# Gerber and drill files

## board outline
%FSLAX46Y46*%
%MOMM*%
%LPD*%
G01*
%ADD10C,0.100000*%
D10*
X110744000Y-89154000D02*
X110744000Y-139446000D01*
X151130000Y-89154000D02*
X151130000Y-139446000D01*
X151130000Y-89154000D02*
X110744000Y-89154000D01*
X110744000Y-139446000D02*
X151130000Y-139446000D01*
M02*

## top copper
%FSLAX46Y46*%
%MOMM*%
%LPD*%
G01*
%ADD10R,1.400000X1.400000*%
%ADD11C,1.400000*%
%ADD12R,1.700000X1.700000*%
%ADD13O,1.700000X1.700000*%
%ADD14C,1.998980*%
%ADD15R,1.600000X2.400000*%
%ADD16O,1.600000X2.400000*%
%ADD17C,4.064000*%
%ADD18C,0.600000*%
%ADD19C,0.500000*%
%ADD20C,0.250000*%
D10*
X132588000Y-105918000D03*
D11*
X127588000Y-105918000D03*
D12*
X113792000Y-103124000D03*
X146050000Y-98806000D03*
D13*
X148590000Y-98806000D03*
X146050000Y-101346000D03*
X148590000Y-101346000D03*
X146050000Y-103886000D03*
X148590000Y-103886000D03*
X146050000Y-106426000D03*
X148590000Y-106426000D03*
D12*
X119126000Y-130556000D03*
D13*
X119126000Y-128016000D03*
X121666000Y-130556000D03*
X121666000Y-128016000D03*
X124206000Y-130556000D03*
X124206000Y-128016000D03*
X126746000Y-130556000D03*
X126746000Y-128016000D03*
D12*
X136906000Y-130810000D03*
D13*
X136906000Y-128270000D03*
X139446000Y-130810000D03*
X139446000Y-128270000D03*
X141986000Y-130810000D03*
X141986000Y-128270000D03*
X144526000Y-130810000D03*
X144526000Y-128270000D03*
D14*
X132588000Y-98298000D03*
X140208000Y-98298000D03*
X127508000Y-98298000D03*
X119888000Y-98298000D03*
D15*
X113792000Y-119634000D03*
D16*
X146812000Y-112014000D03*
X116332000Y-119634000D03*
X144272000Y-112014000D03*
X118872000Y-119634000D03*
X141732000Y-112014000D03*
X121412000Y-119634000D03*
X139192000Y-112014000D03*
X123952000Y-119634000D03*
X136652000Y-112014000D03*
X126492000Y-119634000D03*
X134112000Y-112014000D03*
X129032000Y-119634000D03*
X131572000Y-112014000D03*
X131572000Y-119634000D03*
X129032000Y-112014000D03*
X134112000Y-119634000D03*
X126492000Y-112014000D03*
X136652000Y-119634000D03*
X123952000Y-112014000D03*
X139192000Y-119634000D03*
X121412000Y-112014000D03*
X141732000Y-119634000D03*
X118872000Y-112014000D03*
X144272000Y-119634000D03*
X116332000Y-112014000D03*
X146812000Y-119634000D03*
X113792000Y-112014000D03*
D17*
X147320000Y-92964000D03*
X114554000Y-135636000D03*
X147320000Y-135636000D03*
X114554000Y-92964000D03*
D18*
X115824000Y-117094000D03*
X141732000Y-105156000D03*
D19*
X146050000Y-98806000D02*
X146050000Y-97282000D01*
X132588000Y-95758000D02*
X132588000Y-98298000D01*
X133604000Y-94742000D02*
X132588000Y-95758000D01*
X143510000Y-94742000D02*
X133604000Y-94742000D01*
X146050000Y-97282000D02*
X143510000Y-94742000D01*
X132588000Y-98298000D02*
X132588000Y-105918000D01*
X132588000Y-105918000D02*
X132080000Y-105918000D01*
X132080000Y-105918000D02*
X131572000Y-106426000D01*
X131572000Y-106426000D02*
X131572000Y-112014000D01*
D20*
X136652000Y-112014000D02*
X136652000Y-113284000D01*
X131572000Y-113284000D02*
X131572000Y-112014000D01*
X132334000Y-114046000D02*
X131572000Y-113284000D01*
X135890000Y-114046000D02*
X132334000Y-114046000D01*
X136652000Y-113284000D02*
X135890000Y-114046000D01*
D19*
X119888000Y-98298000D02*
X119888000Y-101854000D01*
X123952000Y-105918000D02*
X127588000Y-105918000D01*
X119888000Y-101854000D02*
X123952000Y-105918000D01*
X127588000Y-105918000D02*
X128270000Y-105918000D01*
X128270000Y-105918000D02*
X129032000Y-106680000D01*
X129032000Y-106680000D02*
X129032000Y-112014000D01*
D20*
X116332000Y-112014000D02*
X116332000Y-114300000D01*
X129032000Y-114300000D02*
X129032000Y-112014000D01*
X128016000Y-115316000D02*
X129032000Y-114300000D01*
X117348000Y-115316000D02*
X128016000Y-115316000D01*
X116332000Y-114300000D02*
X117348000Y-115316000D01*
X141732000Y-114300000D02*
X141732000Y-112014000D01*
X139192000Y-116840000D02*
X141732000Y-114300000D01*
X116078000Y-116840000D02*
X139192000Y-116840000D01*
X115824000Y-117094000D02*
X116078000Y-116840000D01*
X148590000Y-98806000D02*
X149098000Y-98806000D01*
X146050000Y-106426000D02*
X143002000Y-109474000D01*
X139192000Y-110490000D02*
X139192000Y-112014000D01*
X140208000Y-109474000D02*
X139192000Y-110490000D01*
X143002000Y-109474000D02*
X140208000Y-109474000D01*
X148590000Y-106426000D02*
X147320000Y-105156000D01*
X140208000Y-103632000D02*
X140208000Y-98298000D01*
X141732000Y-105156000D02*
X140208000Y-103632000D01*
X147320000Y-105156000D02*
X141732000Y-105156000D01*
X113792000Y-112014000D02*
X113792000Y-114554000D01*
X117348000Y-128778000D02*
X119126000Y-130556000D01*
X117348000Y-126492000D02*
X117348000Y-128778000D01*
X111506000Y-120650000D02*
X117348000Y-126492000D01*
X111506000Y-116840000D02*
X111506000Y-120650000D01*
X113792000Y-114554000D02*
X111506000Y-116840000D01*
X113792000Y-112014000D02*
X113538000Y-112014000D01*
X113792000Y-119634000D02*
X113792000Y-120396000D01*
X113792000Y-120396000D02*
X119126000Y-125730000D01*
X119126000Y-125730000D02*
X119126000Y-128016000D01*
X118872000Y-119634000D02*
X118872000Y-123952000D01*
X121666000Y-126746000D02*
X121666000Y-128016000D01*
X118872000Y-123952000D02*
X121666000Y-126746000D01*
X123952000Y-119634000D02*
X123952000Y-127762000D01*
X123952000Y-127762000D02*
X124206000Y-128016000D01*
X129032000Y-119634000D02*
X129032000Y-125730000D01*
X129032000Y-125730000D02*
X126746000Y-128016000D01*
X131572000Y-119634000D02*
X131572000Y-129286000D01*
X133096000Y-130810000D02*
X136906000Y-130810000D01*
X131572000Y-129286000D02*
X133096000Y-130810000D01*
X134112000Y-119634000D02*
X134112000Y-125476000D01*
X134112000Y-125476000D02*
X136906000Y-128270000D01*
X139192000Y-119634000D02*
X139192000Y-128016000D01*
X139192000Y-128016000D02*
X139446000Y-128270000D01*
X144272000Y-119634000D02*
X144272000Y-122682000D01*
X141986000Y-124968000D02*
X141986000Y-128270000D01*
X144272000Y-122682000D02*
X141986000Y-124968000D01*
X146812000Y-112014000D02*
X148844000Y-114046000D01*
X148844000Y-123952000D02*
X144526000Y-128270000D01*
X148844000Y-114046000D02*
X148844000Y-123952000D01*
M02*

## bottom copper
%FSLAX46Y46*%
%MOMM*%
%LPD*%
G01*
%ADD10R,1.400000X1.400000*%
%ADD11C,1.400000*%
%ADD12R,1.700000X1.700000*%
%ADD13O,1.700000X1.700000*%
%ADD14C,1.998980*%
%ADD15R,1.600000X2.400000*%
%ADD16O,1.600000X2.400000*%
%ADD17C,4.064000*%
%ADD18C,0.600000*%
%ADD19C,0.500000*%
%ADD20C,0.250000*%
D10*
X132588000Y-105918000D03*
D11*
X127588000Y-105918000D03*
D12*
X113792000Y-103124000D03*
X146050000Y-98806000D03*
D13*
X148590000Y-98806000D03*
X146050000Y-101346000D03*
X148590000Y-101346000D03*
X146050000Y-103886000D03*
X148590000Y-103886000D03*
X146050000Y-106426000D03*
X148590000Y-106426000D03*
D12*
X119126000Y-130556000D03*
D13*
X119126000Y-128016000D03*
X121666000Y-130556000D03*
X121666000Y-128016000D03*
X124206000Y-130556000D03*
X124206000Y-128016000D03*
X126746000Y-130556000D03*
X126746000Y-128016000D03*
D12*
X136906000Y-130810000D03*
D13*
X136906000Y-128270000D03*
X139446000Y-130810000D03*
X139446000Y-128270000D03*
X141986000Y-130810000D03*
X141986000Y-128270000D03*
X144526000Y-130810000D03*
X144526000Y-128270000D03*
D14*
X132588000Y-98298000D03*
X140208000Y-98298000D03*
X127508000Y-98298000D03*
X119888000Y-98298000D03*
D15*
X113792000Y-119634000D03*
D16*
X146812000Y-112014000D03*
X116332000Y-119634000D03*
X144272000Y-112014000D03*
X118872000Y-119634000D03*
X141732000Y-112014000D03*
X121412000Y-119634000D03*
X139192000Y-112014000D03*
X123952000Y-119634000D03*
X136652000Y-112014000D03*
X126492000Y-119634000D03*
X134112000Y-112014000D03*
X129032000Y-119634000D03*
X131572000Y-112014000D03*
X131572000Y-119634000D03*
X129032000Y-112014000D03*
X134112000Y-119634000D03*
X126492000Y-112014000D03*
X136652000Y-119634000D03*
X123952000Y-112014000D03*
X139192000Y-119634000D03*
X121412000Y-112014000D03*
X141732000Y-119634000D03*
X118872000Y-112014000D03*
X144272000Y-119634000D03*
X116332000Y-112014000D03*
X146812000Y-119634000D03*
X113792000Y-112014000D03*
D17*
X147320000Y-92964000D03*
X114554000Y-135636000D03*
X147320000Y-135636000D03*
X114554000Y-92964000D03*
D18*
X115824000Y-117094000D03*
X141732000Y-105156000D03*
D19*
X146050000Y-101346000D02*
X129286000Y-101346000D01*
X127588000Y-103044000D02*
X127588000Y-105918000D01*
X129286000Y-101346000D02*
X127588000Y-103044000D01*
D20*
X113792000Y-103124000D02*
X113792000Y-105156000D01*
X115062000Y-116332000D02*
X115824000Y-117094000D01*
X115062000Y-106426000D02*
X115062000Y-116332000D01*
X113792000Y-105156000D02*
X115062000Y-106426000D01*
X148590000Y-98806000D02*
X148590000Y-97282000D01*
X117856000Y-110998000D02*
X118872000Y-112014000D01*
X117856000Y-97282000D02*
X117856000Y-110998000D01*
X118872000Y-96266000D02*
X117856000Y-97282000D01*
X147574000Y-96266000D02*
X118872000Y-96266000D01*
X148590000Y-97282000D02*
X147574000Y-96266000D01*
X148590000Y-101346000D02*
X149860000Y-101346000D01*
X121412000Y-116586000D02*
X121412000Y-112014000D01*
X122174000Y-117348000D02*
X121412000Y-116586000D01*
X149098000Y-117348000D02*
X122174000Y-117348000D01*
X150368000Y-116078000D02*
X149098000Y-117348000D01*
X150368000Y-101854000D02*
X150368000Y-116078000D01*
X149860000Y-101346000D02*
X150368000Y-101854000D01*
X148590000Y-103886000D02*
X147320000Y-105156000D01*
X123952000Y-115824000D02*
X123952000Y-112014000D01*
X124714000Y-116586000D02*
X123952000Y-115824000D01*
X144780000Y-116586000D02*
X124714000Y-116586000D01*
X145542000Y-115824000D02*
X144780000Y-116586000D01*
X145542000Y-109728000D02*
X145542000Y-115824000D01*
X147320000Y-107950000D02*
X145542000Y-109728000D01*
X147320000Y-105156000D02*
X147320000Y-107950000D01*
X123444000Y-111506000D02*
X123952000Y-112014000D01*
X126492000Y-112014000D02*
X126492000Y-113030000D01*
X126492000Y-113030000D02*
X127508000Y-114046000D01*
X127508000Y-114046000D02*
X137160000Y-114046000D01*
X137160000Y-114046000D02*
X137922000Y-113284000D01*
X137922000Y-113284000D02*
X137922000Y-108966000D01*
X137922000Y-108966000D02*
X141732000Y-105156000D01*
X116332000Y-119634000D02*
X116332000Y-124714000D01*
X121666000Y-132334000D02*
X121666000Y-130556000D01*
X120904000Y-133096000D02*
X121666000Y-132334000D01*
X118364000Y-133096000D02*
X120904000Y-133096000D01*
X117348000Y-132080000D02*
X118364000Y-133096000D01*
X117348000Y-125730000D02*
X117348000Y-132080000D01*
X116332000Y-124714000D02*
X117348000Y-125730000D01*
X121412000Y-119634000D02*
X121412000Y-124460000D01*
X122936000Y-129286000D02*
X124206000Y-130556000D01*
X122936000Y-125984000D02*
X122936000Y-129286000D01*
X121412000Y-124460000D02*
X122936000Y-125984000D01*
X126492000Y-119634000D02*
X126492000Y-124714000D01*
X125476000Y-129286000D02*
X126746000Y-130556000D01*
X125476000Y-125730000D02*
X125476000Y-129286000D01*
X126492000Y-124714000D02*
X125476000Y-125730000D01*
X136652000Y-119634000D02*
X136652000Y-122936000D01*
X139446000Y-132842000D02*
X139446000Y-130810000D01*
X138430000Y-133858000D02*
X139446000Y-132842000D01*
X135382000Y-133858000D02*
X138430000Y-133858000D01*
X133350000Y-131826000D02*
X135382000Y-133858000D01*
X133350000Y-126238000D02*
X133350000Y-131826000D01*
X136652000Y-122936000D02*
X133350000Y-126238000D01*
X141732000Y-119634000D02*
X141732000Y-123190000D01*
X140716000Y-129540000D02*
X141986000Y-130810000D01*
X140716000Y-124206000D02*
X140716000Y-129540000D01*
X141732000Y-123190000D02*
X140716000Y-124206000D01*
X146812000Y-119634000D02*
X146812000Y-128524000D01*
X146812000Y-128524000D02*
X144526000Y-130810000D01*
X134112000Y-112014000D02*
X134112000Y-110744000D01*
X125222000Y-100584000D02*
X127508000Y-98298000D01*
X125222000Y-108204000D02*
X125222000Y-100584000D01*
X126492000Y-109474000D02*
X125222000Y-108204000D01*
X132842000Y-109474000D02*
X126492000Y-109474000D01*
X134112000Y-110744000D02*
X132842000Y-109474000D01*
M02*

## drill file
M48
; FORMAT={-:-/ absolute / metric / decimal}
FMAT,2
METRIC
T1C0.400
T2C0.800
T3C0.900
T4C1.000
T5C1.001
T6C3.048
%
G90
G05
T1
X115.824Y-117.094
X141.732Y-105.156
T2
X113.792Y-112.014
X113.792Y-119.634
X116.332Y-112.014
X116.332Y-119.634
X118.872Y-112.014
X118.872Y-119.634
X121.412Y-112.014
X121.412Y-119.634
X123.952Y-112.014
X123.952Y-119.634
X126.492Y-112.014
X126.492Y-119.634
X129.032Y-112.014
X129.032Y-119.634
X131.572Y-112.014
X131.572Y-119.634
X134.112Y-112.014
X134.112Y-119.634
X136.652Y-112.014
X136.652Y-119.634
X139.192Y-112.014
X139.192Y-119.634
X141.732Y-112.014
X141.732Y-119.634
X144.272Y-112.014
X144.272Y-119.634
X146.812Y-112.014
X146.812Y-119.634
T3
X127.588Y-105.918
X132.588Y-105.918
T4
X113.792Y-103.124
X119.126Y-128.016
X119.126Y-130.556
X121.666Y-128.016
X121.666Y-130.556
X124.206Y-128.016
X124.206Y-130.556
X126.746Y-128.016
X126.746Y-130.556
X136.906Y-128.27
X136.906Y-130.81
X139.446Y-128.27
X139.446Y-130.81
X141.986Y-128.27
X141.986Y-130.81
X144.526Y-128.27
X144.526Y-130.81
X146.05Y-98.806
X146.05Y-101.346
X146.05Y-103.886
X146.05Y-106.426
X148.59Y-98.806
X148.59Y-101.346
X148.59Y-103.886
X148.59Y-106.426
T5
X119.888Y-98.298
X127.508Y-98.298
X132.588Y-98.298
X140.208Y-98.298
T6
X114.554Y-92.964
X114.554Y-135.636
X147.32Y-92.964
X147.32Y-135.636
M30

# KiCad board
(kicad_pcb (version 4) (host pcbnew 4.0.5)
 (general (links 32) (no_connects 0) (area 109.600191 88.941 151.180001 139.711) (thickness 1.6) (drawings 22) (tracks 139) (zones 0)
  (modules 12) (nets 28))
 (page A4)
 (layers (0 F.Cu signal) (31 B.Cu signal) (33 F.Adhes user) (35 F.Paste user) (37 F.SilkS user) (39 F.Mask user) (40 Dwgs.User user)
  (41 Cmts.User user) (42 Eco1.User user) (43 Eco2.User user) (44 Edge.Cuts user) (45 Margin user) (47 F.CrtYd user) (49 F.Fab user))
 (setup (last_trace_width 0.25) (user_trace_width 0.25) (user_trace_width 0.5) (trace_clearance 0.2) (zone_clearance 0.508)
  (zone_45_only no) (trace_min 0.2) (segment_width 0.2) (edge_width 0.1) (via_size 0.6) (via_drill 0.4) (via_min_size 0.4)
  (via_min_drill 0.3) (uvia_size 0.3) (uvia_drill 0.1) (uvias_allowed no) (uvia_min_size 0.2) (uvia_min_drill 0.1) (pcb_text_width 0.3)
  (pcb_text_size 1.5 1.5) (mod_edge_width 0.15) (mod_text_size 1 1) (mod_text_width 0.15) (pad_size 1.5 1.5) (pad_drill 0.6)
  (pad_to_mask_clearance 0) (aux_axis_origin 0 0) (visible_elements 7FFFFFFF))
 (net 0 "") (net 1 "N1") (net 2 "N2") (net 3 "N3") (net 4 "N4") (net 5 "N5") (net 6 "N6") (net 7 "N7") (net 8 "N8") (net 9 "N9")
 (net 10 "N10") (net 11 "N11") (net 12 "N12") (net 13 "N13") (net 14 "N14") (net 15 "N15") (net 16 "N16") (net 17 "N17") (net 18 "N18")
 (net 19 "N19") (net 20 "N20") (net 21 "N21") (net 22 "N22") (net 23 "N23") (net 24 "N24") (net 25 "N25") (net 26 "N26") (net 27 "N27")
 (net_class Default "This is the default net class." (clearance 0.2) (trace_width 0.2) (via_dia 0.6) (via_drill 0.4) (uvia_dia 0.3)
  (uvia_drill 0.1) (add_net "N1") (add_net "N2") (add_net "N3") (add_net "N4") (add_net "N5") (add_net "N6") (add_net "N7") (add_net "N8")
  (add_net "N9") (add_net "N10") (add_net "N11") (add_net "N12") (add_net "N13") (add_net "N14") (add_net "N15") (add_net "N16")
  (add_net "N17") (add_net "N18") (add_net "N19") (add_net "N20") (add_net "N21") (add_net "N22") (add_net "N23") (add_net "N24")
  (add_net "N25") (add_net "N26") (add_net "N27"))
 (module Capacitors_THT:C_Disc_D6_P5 (layer F.Cu) (at 132.588 105.918 180)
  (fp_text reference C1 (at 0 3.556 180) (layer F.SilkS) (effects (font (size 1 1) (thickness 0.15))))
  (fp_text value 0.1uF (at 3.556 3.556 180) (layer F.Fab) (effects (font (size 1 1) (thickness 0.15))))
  (pad 1 thru_hole rect (at 0 0 180) (size 1.4 1.4) (drill 0.9) (layers *.Cu *.Mask) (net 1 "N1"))
  (pad 2 thru_hole circle (at 5 0 180) (size 1.4 1.4) (drill 0.9) (layers *.Cu *.Mask) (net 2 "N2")))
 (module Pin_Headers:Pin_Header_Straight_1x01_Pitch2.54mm (layer F.Cu) (at 113.792 103.124)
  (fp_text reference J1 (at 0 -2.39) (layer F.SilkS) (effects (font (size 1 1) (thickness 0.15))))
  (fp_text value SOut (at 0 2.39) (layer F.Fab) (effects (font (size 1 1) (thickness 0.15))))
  (pad 1 thru_hole rect (at 0 0) (size 1.7 1.7) (drill 1) (layers *.Cu *.Mask) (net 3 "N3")))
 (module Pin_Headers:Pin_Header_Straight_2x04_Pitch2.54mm (layer F.Cu) (at 146.05 98.806)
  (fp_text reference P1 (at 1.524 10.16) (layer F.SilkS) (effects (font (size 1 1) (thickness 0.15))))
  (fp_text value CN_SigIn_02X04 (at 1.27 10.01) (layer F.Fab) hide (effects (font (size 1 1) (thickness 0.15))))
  (pad 1 thru_hole rect (at 0 0) (size 1.7 1.7) (drill 1) (layers *.Cu *.Mask) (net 1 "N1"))
  (pad 2 thru_hole oval (at 2.54 0) (size 1.7 1.7) (drill 1) (layers *.Cu *.Mask) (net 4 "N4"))
  (pad 3 thru_hole oval (at 0 2.54) (size 1.7 1.7) (drill 1) (layers *.Cu *.Mask) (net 2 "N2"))
  (pad 4 thru_hole oval (at 2.54 2.54) (size 1.7 1.7) (drill 1) (layers *.Cu *.Mask) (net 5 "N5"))
  (pad 5 thru_hole oval (at 0 5.08) (size 1.7 1.7) (drill 1) (layers *.Cu *.Mask) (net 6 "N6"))
  (pad 6 thru_hole oval (at 2.54 5.08) (size 1.7 1.7) (drill 1) (layers *.Cu *.Mask) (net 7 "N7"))
  (pad 7 thru_hole oval (at 0 7.62) (size 1.7 1.7) (drill 1) (layers *.Cu *.Mask) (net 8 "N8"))
  (pad 8 thru_hole oval (at 2.54 7.62) (size 1.7 1.7) (drill 1) (layers *.Cu *.Mask) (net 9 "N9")))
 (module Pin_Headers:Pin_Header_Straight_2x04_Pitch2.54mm (layer F.Cu) (at 119.126 130.556 90)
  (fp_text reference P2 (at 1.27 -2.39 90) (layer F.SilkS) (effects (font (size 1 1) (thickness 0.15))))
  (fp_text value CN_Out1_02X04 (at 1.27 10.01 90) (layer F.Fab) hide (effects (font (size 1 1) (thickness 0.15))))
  (pad 1 thru_hole rect (at 0 0 90) (size 1.7 1.7) (drill 1) (layers *.Cu *.Mask) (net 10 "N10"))
  (pad 2 thru_hole oval (at 2.54 0 90) (size 1.7 1.7) (drill 1) (layers *.Cu *.Mask) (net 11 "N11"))
  (pad 3 thru_hole oval (at 0 2.54 90) (size 1.7 1.7) (drill 1) (layers *.Cu *.Mask) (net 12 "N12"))
  (pad 4 thru_hole oval (at 2.54 2.54 90) (size 1.7 1.7) (drill 1) (layers *.Cu *.Mask) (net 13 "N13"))
  (pad 5 thru_hole oval (at 0 5.08 90) (size 1.7 1.7) (drill 1) (layers *.Cu *.Mask) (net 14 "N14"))
  (pad 6 thru_hole oval (at 2.54 5.08 90) (size 1.7 1.7) (drill 1) (layers *.Cu *.Mask) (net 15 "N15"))
  (pad 7 thru_hole oval (at 0 7.62 90) (size 1.7 1.7) (drill 1) (layers *.Cu *.Mask) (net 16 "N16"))
  (pad 8 thru_hole oval (at 2.54 7.62 90) (size 1.7 1.7) (drill 1) (layers *.Cu *.Mask) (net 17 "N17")))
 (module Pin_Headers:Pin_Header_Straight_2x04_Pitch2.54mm (layer F.Cu) (at 136.906 130.81 90)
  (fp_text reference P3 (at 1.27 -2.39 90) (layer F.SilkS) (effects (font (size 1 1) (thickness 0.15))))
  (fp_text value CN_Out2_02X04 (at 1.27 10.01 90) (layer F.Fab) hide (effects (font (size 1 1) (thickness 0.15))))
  (pad 1 thru_hole rect (at 0 0 90) (size 1.7 1.7) (drill 1) (layers *.Cu *.Mask) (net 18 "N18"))
  (pad 2 thru_hole oval (at 2.54 0 90) (size 1.7 1.7) (drill 1) (layers *.Cu *.Mask) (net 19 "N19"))
  (pad 3 thru_hole oval (at 0 2.54 90) (size 1.7 1.7) (drill 1) (layers *.Cu *.Mask) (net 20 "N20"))
  (pad 4 thru_hole oval (at 2.54 2.54 90) (size 1.7 1.7) (drill 1) (layers *.Cu *.Mask) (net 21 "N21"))
  (pad 5 thru_hole oval (at 0 5.08 90) (size 1.7 1.7) (drill 1) (layers *.Cu *.Mask) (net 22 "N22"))
  (pad 6 thru_hole oval (at 2.54 5.08 90) (size 1.7 1.7) (drill 1) (layers *.Cu *.Mask) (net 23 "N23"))
  (pad 7 thru_hole oval (at 0 7.62 90) (size 1.7 1.7) (drill 1) (layers *.Cu *.Mask) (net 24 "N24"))
  (pad 8 thru_hole oval (at 2.54 7.62 90) (size 1.7 1.7) (drill 1) (layers *.Cu *.Mask) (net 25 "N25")))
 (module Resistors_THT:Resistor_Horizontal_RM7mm (layer F.Cu) (at 132.588 98.298)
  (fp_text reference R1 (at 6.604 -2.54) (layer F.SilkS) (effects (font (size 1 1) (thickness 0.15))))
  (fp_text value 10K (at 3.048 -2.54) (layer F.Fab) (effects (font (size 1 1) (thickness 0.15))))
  (pad 1 thru_hole circle (at 0 0) (size 1.99898 1.99898) (drill 1.00076) (layers *.Cu *.SilkS *.Mask) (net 1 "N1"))
  (pad 2 thru_hole circle (at 7.62 0) (size 1.99898 1.99898) (drill 1.00076) (layers *.Cu *.SilkS *.Mask) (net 9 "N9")))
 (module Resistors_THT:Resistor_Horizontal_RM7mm (layer F.Cu) (at 127.508 98.298 180)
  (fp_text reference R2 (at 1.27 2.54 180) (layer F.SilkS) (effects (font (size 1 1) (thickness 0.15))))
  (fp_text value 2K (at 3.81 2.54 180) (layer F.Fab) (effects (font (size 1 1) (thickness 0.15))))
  (pad 1 thru_hole circle (at 0 0 180) (size 1.99898 1.99898) (drill 1.00076) (layers *.Cu *.SilkS *.Mask) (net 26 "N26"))
  (pad 2 thru_hole circle (at 7.62 0 180) (size 1.99898 1.99898) (drill 1.00076) (layers *.Cu *.SilkS *.Mask) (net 2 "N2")))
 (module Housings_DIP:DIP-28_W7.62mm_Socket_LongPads (layer F.Cu) (at 113.792 119.634 90)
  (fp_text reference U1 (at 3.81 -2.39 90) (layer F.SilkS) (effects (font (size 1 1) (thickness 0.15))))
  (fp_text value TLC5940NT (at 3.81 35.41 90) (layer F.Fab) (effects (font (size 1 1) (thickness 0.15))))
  (pad 1 thru_hole rect (at 0 0 90) (size 2.4 1.6) (drill 0.8) (layers *.Cu *.Mask) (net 11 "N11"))
  (pad 15 thru_hole oval (at 7.62 33.02 90) (size 2.4 1.6) (drill 0.8) (layers *.Cu *.Mask) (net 25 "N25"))
  (pad 2 thru_hole oval (at 0 2.54 90) (size 2.4 1.6) (drill 0.8) (layers *.Cu *.Mask) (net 12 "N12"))
  (pad 16 thru_hole oval (at 7.62 30.48 90) (size 2.4 1.6) (drill 0.8) (layers *.Cu *.Mask) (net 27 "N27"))
  (pad 3 thru_hole oval (at 0 5.08 90) (size 2.4 1.6) (drill 0.8) (layers *.Cu *.Mask) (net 13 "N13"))
  (pad 17 thru_hole oval (at 7.62 27.94 90) (size 2.4 1.6) (drill 0.8) (layers *.Cu *.Mask) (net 3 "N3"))
  (pad 4 thru_hole oval (at 0 7.62 90) (size 2.4 1.6) (drill 0.8) (layers *.Cu *.Mask) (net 14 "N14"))
  (pad 18 thru_hole oval (at 7.62 25.4 90) (size 2.4 1.6) (drill 0.8) (layers *.Cu *.Mask) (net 8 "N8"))
  (pad 5 thru_hole oval (at 0 10.16 90) (size 2.4 1.6) (drill 0.8) (layers *.Cu *.Mask) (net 15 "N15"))
  (pad 19 thru_hole oval (at 7.62 22.86 90) (size 2.4 1.6) (drill 0.8) (layers *.Cu *.Mask) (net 1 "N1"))
  (pad 6 thru_hole oval (at 0 12.7 90) (size 2.4 1.6) (drill 0.8) (layers *.Cu *.Mask) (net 16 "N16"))
  (pad 20 thru_hole oval (at 7.62 20.32 90) (size 2.4 1.6) (drill 0.8) (layers *.Cu *.Mask) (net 26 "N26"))
  (pad 7 thru_hole oval (at 0 15.24 90) (size 2.4 1.6) (drill 0.8) (layers *.Cu *.Mask) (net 17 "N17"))
  (pad 21 thru_hole oval (at 7.62 17.78 90) (size 2.4 1.6) (drill 0.8) (layers *.Cu *.Mask) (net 1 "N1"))
  (pad 8 thru_hole oval (at 0 17.78 90) (size 2.4 1.6) (drill 0.8) (layers *.Cu *.Mask) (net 18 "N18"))
  (pad 22 thru_hole oval (at 7.62 15.24 90) (size 2.4 1.6) (drill 0.8) (layers *.Cu *.Mask) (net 2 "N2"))
  (pad 9 thru_hole oval (at 0 20.32 90) (size 2.4 1.6) (drill 0.8) (layers *.Cu *.Mask) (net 19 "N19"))
  (pad 23 thru_hole oval (at 7.62 12.7 90) (size 2.4 1.6) (drill 0.8) (layers *.Cu *.Mask) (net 9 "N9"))
  (pad 10 thru_hole oval (at 0 22.86 90) (size 2.4 1.6) (drill 0.8) (layers *.Cu *.Mask) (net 20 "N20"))
  (pad 24 thru_hole oval (at 7.62 10.16 90) (size 2.4 1.6) (drill 0.8) (layers *.Cu *.Mask) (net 7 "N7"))
  (pad 11 thru_hole oval (at 0 25.4 90) (size 2.4 1.6) (drill 0.8) (layers *.Cu *.Mask) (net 21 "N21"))
  (pad 25 thru_hole oval (at 7.62 7.62 90) (size 2.4 1.6) (drill 0.8) (layers *.Cu *.Mask) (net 5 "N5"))
  (pad 12 thru_hole oval (at 0 27.94 90) (size 2.4 1.6) (drill 0.8) (layers *.Cu *.Mask) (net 22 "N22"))
  (pad 26 thru_hole oval (at 7.62 5.08 90) (size 2.4 1.6) (drill 0.8) (layers *.Cu *.Mask) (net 4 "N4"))
  (pad 13 thru_hole oval (at 0 30.48 90) (size 2.4 1.6) (drill 0.8) (layers *.Cu *.Mask) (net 23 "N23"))
  (pad 27 thru_hole oval (at 7.62 2.54 90) (size 2.4 1.6) (drill 0.8) (layers *.Cu *.Mask) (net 2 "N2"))
  (pad 14 thru_hole oval (at 0 33.02 90) (size 2.4 1.6) (drill 0.8) (layers *.Cu *.Mask) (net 24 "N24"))
  (pad 28 thru_hole oval (at 7.62 0 90) (size 2.4 1.6) (drill 0.8) (layers *.Cu *.Mask) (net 10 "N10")))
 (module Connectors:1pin (layer F.Cu) (at 147.32 92.964)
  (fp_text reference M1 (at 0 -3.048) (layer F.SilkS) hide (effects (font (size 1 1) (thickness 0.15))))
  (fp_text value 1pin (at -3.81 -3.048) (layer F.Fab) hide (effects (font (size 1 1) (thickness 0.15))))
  (pad 1 thru_hole circle (at 0 0) (size 4.064 4.064) (drill 3.048) (layers *.Cu *.Mask)))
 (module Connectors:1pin (layer F.Cu) (at 114.554 135.636)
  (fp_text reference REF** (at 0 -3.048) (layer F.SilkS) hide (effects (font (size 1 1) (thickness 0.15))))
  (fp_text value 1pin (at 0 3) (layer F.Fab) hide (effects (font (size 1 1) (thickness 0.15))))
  (pad 1 thru_hole circle (at 0 0) (size 4.064 4.064) (drill 3.048) (layers *.Cu *.Mask)))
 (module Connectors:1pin (layer F.Cu) (at 147.32 135.636)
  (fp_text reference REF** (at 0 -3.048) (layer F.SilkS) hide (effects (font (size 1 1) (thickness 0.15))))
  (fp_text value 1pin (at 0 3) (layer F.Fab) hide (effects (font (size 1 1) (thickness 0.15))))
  (pad 1 thru_hole circle (at 0 0) (size 4.064 4.064) (drill 3.048) (layers *.Cu *.Mask)))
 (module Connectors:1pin (layer F.Cu) (at 114.554 92.964)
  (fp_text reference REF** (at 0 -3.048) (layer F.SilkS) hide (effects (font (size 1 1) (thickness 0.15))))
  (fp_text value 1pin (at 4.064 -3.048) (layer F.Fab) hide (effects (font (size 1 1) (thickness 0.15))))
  (pad 1 thru_hole circle (at 0 0) (size 4.064 4.064) (drill 3.048) (layers *.Cu *.Mask)))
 (gr_line (start 110.744 89.154) (end 110.744 139.446) (angle 90) (layer Edge.Cuts) (width 0.1))
 (gr_line (start 151.13 89.154) (end 151.13 139.446) (angle 90) (layer Edge.Cuts) (width 0.1))
 (gr_line (start 151.13 89.154) (end 110.744 89.154) (angle 90) (layer Edge.Cuts) (width 0.1))
 (gr_line (start 110.744 139.446) (end 151.13 139.446) (angle 90) (layer Edge.Cuts) (width 0.1))
 (segment (start 146.05 98.806) (end 146.05 97.282) (width 0.5) (layer F.Cu) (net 1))
 (segment (start 132.588 95.758) (end 132.588 98.298) (width 0.5) (layer F.Cu) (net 1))
 (segment (start 133.604 94.742) (end 132.588 95.758) (width 0.5) (layer F.Cu) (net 1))
 (segment (start 143.51 94.742) (end 133.604 94.742) (width 0.5) (layer F.Cu) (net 1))
 (segment (start 146.05 97.282) (end 143.51 94.742) (width 0.5) (layer F.Cu) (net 1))
 (segment (start 132.588 98.298) (end 132.588 105.918) (width 0.5) (layer F.Cu) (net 1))
 (segment (start 132.588 105.918) (end 132.08 105.918) (width 0.5) (layer F.Cu) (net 1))
 (segment (start 132.08 105.918) (end 131.572 106.426) (width 0.5) (layer F.Cu) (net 1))
 (segment (start 131.572 106.426) (end 131.572 112.014) (width 0.5) (layer F.Cu) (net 1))
 (segment (start 136.652 112.014) (end 136.652 113.284) (width 0.25) (layer F.Cu) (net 1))
 (segment (start 131.572 113.284) (end 131.572 112.014) (width 0.25) (layer F.Cu) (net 1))
 (segment (start 132.334 114.046) (end 131.572 113.284) (width 0.25) (layer F.Cu) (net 1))
 (segment (start 135.89 114.046) (end 132.334 114.046) (width 0.25) (layer F.Cu) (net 1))
 (segment (start 136.652 113.284) (end 135.89 114.046) (width 0.25) (layer F.Cu) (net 1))
 (segment (start 146.05 101.346) (end 129.286 101.346) (width 0.5) (layer B.Cu) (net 2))
 (segment (start 127.588 103.044) (end 127.588 105.918) (width 0.5) (layer B.Cu) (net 2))
 (segment (start 129.286 101.346) (end 127.588 103.044) (width 0.5) (layer B.Cu) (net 2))
 (segment (start 119.888 98.298) (end 119.888 101.854) (width 0.5) (layer F.Cu) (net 2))
 (segment (start 123.952 105.918) (end 127.588 105.918) (width 0.5) (layer F.Cu) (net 2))
 (segment (start 119.888 101.854) (end 123.952 105.918) (width 0.5) (layer F.Cu) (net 2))
 (segment (start 127.588 105.918) (end 128.27 105.918) (width 0.5) (layer F.Cu) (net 2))
 (segment (start 128.27 105.918) (end 129.032 106.68) (width 0.5) (layer F.Cu) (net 2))
 (segment (start 129.032 106.68) (end 129.032 112.014) (width 0.5) (layer F.Cu) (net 2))
 (segment (start 116.332 112.014) (end 116.332 114.3) (width 0.25) (layer F.Cu) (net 2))
 (segment (start 129.032 114.3) (end 129.032 112.014) (width 0.25) (layer F.Cu) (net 2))
 (segment (start 128.016 115.316) (end 129.032 114.3) (width 0.25) (layer F.Cu) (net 2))
 (segment (start 117.348 115.316) (end 128.016 115.316) (width 0.25) (layer F.Cu) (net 2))
 (segment (start 116.332 114.3) (end 117.348 115.316) (width 0.25) (layer F.Cu) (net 2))
 (segment (start 113.792 103.124) (end 113.792 105.156) (width 0.25) (layer B.Cu) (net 3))
 (segment (start 141.732 114.3) (end 141.732 112.014) (width 0.25) (layer F.Cu) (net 3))
 (segment (start 139.192 116.84) (end 141.732 114.3) (width 0.25) (layer F.Cu) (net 3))
 (segment (start 116.078 116.84) (end 139.192 116.84) (width 0.25) (layer F.Cu) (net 3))
 (segment (start 115.824 117.094) (end 116.078 116.84) (width 0.25) (layer F.Cu) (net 3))
 (via (at 115.824 117.094) (size 0.6) (drill 0.4) (layers F.Cu B.Cu) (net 3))
 (segment (start 115.062 116.332) (end 115.824 117.094) (width 0.25) (layer B.Cu) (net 3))
 (segment (start 115.062 106.426) (end 115.062 116.332) (width 0.25) (layer B.Cu) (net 3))
 (segment (start 113.792 105.156) (end 115.062 106.426) (width 0.25) (layer B.Cu) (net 3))
 (segment (start 148.59 98.806) (end 148.59 97.282) (width 0.25) (layer B.Cu) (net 4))
 (segment (start 117.856 110.998) (end 118.872 112.014) (width 0.25) (layer B.Cu) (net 4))
 (segment (start 117.856 97.282) (end 117.856 110.998) (width 0.25) (layer B.Cu) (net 4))
 (segment (start 118.872 96.266) (end 117.856 97.282) (width 0.25) (layer B.Cu) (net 4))
 (segment (start 147.574 96.266) (end 118.872 96.266) (width 0.25) (layer B.Cu) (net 4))
 (segment (start 148.59 97.282) (end 147.574 96.266) (width 0.25) (layer B.Cu) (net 4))
 (segment (start 148.59 98.806) (end 149.098 98.806) (width 0.25) (layer F.Cu) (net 4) (status 30))
 (segment (start 148.59 101.346) (end 149.86 101.346) (width 0.25) (layer B.Cu) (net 5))
 (segment (start 121.412 116.586) (end 121.412 112.014) (width 0.25) (layer B.Cu) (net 5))
 (segment (start 122.174 117.348) (end 121.412 116.586) (width 0.25) (layer B.Cu) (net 5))
 (segment (start 149.098 117.348) (end 122.174 117.348) (width 0.25) (layer B.Cu) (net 5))
 (segment (start 150.368 116.078) (end 149.098 117.348) (width 0.25) (layer B.Cu) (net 5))
 (segment (start 150.368 101.854) (end 150.368 116.078) (width 0.25) (layer B.Cu) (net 5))
 (segment (start 149.86 101.346) (end 150.368 101.854) (width 0.25) (layer B.Cu) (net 5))
 (segment (start 148.59 103.886) (end 147.32 105.156) (width 0.25) (layer B.Cu) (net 7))
 (segment (start 123.952 115.824) (end 123.952 112.014) (width 0.25) (layer B.Cu) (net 7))
 (segment (start 124.714 116.586) (end 123.952 115.824) (width 0.25) (layer B.Cu) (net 7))
 (segment (start 144.78 116.586) (end 124.714 116.586) (width 0.25) (layer B.Cu) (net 7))
 (segment (start 145.542 115.824) (end 144.78 116.586) (width 0.25) (layer B.Cu) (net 7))
 (segment (start 145.542 109.728) (end 145.542 115.824) (width 0.25) (layer B.Cu) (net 7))
 (segment (start 147.32 107.95) (end 145.542 109.728) (width 0.25) (layer B.Cu) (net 7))
 (segment (start 147.32 105.156) (end 147.32 107.95) (width 0.25) (layer B.Cu) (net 7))
 (segment (start 123.444 111.506) (end 123.952 112.014) (width 0.25) (layer B.Cu) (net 7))
 (segment (start 146.05 106.426) (end 143.002 109.474) (width 0.25) (layer F.Cu) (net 8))
 (segment (start 139.192 110.49) (end 139.192 112.014) (width 0.25) (layer F.Cu) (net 8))
 (segment (start 140.208 109.474) (end 139.192 110.49) (width 0.25) (layer F.Cu) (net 8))
 (segment (start 143.002 109.474) (end 140.208 109.474) (width 0.25) (layer F.Cu) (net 8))
 (segment (start 126.492 112.014) (end 126.492 113.03) (width 0.25) (layer B.Cu) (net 9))
 (segment (start 126.492 113.03) (end 127.508 114.046) (width 0.25) (layer B.Cu) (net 9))
 (segment (start 127.508 114.046) (end 137.16 114.046) (width 0.25) (layer B.Cu) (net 9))
 (segment (start 137.16 114.046) (end 137.922 113.284) (width 0.25) (layer B.Cu) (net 9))
 (segment (start 137.922 113.284) (end 137.922 108.966) (width 0.25) (layer B.Cu) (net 9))
 (segment (start 137.922 108.966) (end 141.732 105.156) (width 0.25) (layer B.Cu) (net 9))
 (via (at 141.732 105.156) (size 0.6) (drill 0.4) (layers F.Cu B.Cu) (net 9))
 (segment (start 148.59 106.426) (end 147.32 105.156) (width 0.25) (layer F.Cu) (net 9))
 (segment (start 140.208 103.632) (end 140.208 98.298) (width 0.25) (layer F.Cu) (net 9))
 (segment (start 141.732 105.156) (end 140.208 103.632) (width 0.25) (layer F.Cu) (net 9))
 (segment (start 147.32 105.156) (end 141.732 105.156) (width 0.25) (layer F.Cu) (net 9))
 (segment (start 113.792 112.014) (end 113.792 114.554) (width 0.25) (layer F.Cu) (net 10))
 (segment (start 117.348 128.778) (end 119.126 130.556) (width 0.25) (layer F.Cu) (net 10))
 (segment (start 117.348 126.492) (end 117.348 128.778) (width 0.25) (layer F.Cu) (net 10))
 (segment (start 111.506 120.65) (end 117.348 126.492) (width 0.25) (layer F.Cu) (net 10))
 (segment (start 111.506 116.84) (end 111.506 120.65) (width 0.25) (layer F.Cu) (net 10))
 (segment (start 113.792 114.554) (end 111.506 116.84) (width 0.25) (layer F.Cu) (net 10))
 (segment (start 113.792 112.014) (end 113.538 112.014) (width 0.25) (layer F.Cu) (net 10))
 (segment (start 113.792 119.634) (end 113.792 120.396) (width 0.25) (layer F.Cu) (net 11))
 (segment (start 113.792 120.396) (end 119.126 125.73) (width 0.25) (layer F.Cu) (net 11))
 (segment (start 119.126 125.73) (end 119.126 128.016) (width 0.25) (layer F.Cu) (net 11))
 (segment (start 116.332 119.634) (end 116.332 124.714) (width 0.25) (layer B.Cu) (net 12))
 (segment (start 121.666 132.334) (end 121.666 130.556) (width 0.25) (layer B.Cu) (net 12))
 (segment (start 120.904 133.096) (end 121.666 132.334) (width 0.25) (layer B.Cu) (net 12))
 (segment (start 118.364 133.096) (end 120.904 133.096) (width 0.25) (layer B.Cu) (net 12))
 (segment (start 117.348 132.08) (end 118.364 133.096) (width 0.25) (layer B.Cu) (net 12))
 (segment (start 117.348 125.73) (end 117.348 132.08) (width 0.25) (layer B.Cu) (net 12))
 (segment (start 116.332 124.714) (end 117.348 125.73) (width 0.25) (layer B.Cu) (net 12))
 (segment (start 118.872 119.634) (end 118.872 123.952) (width 0.25) (layer F.Cu) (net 13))
 (segment (start 121.666 126.746) (end 121.666 128.016) (width 0.25) (layer F.Cu) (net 13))
 (segment (start 118.872 123.952) (end 121.666 126.746) (width 0.25) (layer F.Cu) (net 13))
 (segment (start 121.412 119.634) (end 121.412 124.46) (width 0.25) (layer B.Cu) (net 14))
 (segment (start 122.936 129.286) (end 124.206 130.556) (width 0.25) (layer B.Cu) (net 14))
 (segment (start 122.936 125.984) (end 122.936 129.286) (width 0.25) (layer B.Cu) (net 14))
 (segment (start 121.412 124.46) (end 122.936 125.984) (width 0.25) (layer B.Cu) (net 14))
 (segment (start 123.952 119.634) (end 123.952 127.762) (width 0.25) (layer F.Cu) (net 15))
 (segment (start 123.952 127.762) (end 124.206 128.016) (width 0.25) (layer F.Cu) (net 15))
 (segment (start 126.492 119.634) (end 126.492 124.714) (width 0.25) (layer B.Cu) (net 16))
 (segment (start 125.476 129.286) (end 126.746 130.556) (width 0.25) (layer B.Cu) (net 16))
 (segment (start 125.476 125.73) (end 125.476 129.286) (width 0.25) (layer B.Cu) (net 16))
 (segment (start 126.492 124.714) (end 125.476 125.73) (width 0.25) (layer B.Cu) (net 16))
 (segment (start 129.032 119.634) (end 129.032 125.73) (width 0.25) (layer F.Cu) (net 17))
 (segment (start 129.032 125.73) (end 126.746 128.016) (width 0.25) (layer F.Cu) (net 17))
 (segment (start 131.572 119.634) (end 131.572 129.286) (width 0.25) (layer F.Cu) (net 18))
 (segment (start 133.096 130.81) (end 136.906 130.81) (width 0.25) (layer F.Cu) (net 18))
 (segment (start 131.572 129.286) (end 133.096 130.81) (width 0.25) (layer F.Cu) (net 18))
 (segment (start 134.112 119.634) (end 134.112 125.476) (width 0.25) (layer F.Cu) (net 19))
 (segment (start 134.112 125.476) (end 136.906 128.27) (width 0.25) (layer F.Cu) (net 19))
 (segment (start 136.652 119.634) (end 136.652 122.936) (width 0.25) (layer B.Cu) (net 20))
 (segment (start 139.446 132.842) (end 139.446 130.81) (width 0.25) (layer B.Cu) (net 20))
 (segment (start 138.43 133.858) (end 139.446 132.842) (width 0.25) (layer B.Cu) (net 20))
 (segment (start 135.382 133.858) (end 138.43 133.858) (width 0.25) (layer B.Cu) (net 20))
 (segment (start 133.35 131.826) (end 135.382 133.858) (width 0.25) (layer B.Cu) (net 20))
 (segment (start 133.35 126.238) (end 133.35 131.826) (width 0.25) (layer B.Cu) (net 20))
 (segment (start 136.652 122.936) (end 133.35 126.238) (width 0.25) (layer B.Cu) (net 20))
 (segment (start 139.192 119.634) (end 139.192 128.016) (width 0.25) (layer F.Cu) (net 21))
 (segment (start 139.192 128.016) (end 139.446 128.27) (width 0.25) (layer F.Cu) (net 21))
 (segment (start 141.732 119.634) (end 141.732 123.19) (width 0.25) (layer B.Cu) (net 22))
 (segment (start 140.716 129.54) (end 141.986 130.81) (width 0.25) (layer B.Cu) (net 22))
 (segment (start 140.716 124.206) (end 140.716 129.54) (width 0.25) (layer B.Cu) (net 22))
 (segment (start 141.732 123.19) (end 140.716 124.206) (width 0.25) (layer B.Cu) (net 22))
 (segment (start 144.272 119.634) (end 144.272 122.682) (width 0.25) (layer F.Cu) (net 23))
 (segment (start 141.986 124.968) (end 141.986 128.27) (width 0.25) (layer F.Cu) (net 23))
 (segment (start 144.272 122.682) (end 141.986 124.968) (width 0.25) (layer F.Cu) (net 23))
 (segment (start 146.812 119.634) (end 146.812 128.524) (width 0.25) (layer B.Cu) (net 24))
 (segment (start 146.812 128.524) (end 144.526 130.81) (width 0.25) (layer B.Cu) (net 24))
 (segment (start 146.812 112.014) (end 148.844 114.046) (width 0.25) (layer F.Cu) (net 25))
 (segment (start 148.844 123.952) (end 144.526 128.27) (width 0.25) (layer F.Cu) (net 25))
 (segment (start 148.844 114.046) (end 148.844 123.952) (width 0.25) (layer F.Cu) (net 25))
 (segment (start 134.112 112.014) (end 134.112 110.744) (width 0.25) (layer B.Cu) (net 26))
 (segment (start 125.222 100.584) (end 127.508 98.298) (width 0.25) (layer B.Cu) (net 26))
 (segment (start 125.222 108.204) (end 125.222 100.584) (width 0.25) (layer B.Cu) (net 26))
 (segment (start 126.492 109.474) (end 125.222 108.204) (width 0.25) (layer B.Cu) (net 26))
 (segment (start 132.842 109.474) (end 126.492 109.474) (width 0.25) (layer B.Cu) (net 26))
 (segment (start 134.112 110.744) (end 132.842 109.474) (width 0.25) (layer B.Cu) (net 26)))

